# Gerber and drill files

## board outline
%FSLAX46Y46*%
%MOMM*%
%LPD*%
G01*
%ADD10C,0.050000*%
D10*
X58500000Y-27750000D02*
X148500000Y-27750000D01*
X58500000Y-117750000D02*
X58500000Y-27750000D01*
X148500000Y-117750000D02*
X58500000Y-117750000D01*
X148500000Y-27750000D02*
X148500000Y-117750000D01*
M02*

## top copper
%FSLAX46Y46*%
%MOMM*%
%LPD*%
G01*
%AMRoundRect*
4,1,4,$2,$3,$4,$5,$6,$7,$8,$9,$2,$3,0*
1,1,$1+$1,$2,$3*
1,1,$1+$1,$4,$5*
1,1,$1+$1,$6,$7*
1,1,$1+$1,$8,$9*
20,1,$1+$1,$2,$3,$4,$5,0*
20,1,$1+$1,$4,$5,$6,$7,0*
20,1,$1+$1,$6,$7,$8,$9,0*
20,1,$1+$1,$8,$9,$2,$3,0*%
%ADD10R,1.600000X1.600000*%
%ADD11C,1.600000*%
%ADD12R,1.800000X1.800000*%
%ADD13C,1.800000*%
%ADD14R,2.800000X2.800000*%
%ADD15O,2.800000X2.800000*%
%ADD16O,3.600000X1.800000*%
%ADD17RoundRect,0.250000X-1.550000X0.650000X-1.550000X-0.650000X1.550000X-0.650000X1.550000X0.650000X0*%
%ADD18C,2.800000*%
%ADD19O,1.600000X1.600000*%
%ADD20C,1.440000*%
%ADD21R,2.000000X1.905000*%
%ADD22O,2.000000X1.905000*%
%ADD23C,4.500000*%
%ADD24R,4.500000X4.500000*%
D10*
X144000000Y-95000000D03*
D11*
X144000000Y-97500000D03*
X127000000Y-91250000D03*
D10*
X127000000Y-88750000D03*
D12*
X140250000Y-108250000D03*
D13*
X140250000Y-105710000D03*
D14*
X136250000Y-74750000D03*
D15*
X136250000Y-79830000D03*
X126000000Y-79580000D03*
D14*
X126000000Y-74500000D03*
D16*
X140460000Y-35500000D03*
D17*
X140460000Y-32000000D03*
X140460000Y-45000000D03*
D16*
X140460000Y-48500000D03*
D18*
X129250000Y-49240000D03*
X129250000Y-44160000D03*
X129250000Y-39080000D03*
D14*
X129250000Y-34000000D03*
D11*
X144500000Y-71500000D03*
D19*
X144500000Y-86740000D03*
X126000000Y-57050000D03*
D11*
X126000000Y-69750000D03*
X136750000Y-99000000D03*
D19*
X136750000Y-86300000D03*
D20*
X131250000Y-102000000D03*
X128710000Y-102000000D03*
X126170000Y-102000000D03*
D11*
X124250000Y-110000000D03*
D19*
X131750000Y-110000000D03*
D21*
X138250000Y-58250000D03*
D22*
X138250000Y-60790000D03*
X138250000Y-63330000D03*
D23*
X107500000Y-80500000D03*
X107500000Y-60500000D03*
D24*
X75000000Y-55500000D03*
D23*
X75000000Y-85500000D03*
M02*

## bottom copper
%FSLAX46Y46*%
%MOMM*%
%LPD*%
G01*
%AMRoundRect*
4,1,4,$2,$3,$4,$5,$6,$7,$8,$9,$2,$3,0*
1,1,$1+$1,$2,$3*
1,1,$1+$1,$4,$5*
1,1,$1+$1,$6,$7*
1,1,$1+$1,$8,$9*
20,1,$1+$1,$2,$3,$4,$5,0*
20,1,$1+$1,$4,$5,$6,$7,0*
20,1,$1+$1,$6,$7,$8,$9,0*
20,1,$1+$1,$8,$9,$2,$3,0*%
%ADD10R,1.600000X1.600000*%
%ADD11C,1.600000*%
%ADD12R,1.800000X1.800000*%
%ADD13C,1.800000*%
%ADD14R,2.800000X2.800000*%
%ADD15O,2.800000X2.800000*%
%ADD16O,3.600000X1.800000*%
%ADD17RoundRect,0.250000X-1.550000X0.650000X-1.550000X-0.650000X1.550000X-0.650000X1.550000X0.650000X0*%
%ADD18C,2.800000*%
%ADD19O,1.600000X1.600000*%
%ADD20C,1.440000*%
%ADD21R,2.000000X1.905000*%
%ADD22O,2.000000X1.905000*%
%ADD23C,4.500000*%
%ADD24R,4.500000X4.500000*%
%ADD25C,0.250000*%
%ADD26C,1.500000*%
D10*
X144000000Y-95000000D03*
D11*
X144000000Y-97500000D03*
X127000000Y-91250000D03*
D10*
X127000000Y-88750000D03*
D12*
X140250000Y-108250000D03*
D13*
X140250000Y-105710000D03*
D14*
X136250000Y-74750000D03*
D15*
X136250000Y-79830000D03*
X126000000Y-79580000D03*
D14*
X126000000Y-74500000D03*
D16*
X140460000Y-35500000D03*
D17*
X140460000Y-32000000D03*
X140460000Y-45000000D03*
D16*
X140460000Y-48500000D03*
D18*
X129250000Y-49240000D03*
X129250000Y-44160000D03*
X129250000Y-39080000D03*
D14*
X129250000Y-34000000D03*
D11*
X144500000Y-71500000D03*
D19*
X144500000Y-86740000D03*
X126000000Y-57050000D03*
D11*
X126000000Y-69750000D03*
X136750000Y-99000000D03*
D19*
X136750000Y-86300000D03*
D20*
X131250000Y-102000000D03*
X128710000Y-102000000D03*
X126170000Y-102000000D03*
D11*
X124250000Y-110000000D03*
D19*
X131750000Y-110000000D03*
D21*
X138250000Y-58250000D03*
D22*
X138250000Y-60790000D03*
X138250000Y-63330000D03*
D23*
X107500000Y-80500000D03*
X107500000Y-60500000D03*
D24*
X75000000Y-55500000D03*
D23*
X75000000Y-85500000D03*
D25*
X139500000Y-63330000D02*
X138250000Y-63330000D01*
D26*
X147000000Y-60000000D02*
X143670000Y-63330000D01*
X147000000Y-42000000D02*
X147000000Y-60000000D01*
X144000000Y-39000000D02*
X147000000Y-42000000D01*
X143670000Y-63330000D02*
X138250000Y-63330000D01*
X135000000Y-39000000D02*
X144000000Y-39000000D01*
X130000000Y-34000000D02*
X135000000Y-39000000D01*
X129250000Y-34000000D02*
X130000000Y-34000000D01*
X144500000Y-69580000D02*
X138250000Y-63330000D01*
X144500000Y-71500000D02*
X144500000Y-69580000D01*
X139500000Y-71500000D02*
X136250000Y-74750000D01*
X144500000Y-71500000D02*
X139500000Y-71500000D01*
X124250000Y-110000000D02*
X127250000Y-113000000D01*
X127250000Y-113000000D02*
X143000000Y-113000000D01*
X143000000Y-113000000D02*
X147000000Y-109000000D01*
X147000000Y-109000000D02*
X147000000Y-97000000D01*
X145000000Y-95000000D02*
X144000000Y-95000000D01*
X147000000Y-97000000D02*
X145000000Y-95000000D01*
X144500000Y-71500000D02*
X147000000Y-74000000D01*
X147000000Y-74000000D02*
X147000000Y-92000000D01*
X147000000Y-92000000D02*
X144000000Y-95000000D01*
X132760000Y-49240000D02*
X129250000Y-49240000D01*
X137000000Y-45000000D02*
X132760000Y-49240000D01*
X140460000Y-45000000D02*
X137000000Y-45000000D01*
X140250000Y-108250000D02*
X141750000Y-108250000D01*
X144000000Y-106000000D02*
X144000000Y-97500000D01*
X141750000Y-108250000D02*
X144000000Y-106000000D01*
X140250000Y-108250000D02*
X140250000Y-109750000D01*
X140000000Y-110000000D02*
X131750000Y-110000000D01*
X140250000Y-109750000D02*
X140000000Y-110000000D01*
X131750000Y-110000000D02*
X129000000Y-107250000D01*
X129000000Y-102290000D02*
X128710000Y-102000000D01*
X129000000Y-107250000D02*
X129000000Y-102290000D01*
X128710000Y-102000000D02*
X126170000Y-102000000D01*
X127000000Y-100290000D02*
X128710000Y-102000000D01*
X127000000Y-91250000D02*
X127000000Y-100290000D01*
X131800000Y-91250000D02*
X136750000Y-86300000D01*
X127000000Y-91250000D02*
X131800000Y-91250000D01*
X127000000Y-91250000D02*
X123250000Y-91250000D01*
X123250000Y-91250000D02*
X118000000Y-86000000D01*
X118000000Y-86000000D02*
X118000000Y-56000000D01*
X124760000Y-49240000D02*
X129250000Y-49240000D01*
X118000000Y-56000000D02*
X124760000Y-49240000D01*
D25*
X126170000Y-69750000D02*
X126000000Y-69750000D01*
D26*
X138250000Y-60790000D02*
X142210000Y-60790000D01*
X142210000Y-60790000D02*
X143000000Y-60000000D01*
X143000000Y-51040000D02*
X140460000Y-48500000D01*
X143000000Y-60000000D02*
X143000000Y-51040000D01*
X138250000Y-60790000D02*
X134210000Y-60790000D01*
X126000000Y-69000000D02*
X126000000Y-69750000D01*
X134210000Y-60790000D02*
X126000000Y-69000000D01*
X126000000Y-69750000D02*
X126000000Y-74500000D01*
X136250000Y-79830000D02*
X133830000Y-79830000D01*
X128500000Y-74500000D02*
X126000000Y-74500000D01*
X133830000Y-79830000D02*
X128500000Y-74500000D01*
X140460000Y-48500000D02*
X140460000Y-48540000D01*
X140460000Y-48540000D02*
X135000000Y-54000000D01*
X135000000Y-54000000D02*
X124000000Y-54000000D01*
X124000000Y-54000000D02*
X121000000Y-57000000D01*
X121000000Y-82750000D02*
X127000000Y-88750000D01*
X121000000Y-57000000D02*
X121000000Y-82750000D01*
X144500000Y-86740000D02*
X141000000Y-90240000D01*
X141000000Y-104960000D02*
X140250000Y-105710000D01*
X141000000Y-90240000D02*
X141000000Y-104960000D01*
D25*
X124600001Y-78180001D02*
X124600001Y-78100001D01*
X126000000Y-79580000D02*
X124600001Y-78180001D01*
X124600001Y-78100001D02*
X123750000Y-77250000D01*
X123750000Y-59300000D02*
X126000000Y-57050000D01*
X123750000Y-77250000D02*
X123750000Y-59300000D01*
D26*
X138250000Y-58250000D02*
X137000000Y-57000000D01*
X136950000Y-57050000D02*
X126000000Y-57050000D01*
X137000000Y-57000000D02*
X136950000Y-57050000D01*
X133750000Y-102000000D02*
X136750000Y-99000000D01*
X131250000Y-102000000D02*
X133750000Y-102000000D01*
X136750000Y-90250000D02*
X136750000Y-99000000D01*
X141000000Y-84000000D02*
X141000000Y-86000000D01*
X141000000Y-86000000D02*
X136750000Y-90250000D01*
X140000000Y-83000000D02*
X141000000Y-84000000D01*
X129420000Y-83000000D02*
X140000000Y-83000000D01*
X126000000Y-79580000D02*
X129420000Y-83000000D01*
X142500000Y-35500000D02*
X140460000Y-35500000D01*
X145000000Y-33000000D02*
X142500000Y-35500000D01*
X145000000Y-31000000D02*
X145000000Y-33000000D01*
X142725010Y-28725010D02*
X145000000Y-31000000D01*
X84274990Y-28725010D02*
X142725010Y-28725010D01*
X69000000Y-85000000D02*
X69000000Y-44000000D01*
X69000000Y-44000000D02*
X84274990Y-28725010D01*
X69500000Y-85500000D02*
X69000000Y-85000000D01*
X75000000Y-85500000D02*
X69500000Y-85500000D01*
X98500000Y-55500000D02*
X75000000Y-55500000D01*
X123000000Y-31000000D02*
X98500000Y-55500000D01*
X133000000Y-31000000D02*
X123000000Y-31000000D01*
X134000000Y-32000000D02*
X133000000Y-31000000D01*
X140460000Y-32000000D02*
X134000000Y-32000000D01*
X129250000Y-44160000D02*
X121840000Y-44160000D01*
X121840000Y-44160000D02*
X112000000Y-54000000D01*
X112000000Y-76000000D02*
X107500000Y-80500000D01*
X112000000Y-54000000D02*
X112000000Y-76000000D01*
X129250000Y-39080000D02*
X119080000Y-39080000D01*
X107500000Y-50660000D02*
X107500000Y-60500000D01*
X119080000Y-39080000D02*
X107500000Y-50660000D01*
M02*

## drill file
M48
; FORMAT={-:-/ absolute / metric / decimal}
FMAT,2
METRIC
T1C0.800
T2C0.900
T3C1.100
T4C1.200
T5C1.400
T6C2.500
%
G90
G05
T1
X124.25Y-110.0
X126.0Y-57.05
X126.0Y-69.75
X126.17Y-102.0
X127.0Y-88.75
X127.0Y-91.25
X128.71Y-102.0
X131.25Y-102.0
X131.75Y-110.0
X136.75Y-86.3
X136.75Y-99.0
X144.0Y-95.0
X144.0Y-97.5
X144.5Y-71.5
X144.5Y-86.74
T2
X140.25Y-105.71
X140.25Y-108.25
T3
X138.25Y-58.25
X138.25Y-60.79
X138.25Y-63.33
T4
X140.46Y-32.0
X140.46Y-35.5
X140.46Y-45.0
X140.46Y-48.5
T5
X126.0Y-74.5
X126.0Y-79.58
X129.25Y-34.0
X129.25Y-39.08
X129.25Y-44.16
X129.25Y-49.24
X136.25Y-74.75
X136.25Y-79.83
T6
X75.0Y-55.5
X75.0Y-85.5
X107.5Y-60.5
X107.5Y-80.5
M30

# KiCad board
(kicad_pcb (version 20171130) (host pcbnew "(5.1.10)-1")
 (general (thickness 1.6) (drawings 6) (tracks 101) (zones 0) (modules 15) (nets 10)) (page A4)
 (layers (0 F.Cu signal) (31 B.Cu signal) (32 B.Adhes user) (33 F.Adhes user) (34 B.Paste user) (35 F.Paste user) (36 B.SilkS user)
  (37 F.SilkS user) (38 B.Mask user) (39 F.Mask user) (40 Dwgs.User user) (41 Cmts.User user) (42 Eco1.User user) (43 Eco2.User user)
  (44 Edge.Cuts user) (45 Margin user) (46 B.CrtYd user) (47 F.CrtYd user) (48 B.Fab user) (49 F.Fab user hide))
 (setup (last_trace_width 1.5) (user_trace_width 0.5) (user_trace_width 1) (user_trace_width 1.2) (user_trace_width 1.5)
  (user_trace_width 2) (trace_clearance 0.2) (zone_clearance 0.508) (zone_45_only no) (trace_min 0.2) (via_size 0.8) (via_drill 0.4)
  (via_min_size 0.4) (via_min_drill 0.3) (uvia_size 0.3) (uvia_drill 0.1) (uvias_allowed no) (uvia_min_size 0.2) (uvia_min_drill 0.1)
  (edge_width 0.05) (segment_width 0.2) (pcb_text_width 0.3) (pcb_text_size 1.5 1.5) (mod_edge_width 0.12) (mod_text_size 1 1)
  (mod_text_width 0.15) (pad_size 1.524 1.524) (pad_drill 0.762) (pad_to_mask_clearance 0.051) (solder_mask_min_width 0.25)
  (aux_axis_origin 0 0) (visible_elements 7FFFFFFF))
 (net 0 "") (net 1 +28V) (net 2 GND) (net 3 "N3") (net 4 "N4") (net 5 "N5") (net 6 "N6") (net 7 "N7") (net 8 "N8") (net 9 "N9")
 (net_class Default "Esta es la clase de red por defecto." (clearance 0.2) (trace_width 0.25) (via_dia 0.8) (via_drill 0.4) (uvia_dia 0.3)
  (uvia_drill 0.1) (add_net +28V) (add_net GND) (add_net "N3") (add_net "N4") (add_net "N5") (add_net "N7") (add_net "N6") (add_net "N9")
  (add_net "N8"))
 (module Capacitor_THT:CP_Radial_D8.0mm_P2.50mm (layer F.Cu) (at 144 95 270)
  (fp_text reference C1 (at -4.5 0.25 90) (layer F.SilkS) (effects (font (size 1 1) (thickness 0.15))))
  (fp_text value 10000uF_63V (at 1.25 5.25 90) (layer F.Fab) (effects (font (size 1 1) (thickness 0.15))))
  (pad 1 thru_hole rect (at 0 0 270) (size 1.6 1.6) (drill 0.8) (layers *.Cu *.Mask) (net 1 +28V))
  (pad 2 thru_hole circle (at 2.5 0 270) (size 1.6 1.6) (drill 0.8) (layers *.Cu *.Mask) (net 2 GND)))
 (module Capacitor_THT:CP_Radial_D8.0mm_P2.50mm (layer F.Cu) (at 127 88.75 270)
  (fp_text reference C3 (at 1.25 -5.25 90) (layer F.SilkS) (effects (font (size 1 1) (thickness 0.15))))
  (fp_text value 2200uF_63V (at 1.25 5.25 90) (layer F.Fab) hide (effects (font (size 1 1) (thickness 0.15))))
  (pad 2 thru_hole circle (at 2.5 0 270) (size 1.6 1.6) (drill 0.8) (layers *.Cu *.Mask) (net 2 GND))
  (pad 1 thru_hole rect (at 0 0 270) (size 1.6 1.6) (drill 0.8) (layers *.Cu *.Mask) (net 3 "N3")))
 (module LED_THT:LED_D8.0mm (layer F.Cu) (at 140.25 108.25 90)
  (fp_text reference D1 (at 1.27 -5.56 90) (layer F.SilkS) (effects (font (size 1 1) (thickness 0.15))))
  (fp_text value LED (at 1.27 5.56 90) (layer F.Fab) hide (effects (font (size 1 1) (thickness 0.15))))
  (pad 1 thru_hole rect (at 0 0 90) (size 1.8 1.8) (drill 0.9) (layers *.Cu *.Mask) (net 2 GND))
  (pad 2 thru_hole circle (at 2.54 0 90) (size 1.8 1.8) (drill 0.9) (layers *.Cu *.Mask) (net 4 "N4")))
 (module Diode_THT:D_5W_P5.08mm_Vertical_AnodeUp (layer F.Cu) (at 136.25 74.75 270)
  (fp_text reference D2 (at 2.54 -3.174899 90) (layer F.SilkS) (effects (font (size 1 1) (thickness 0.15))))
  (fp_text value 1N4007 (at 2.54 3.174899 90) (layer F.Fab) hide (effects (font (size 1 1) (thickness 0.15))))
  (pad 1 thru_hole rect (at 0 0 270) (size 2.8 2.8) (drill 1.4) (layers *.Cu *.Mask) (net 1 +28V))
  (pad 2 thru_hole oval (at 5.08 0 270) (size 2.8 2.8) (drill 1.4) (layers *.Cu *.Mask) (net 3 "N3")))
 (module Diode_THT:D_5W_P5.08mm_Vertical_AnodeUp (layer F.Cu) (at 126 74.5 270)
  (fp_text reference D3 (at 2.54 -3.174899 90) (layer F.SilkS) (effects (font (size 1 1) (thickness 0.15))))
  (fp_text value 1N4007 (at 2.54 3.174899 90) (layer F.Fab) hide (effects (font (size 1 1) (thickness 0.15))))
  (pad 2 thru_hole oval (at 5.08 0 270) (size 2.8 2.8) (drill 1.4) (layers *.Cu *.Mask) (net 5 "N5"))
  (pad 1 thru_hole rect (at 0 0 270) (size 2.8 2.8) (drill 1.4) (layers *.Cu *.Mask) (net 3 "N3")))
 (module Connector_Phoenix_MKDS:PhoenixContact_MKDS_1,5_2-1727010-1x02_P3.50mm (layer F.Cu) (at 143 32 270)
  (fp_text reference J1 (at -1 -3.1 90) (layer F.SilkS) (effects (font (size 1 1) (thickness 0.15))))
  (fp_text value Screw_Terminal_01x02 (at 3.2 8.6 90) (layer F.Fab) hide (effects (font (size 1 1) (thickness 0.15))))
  (pad 2 thru_hole oval (at 3.5 2.54 270) (size 1.8 3.6) (drill 1.2) (layers *.Cu *.Mask) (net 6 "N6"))
  (pad 1 thru_hole roundrect (at 0 2.54 270) (size 1.8 3.6) (drill 1.2) (layers *.Cu *.Mask) (roundrect_rratio 0.138889) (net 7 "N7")))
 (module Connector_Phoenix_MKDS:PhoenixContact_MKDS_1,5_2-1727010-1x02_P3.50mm (layer F.Cu) (at 143 45 270)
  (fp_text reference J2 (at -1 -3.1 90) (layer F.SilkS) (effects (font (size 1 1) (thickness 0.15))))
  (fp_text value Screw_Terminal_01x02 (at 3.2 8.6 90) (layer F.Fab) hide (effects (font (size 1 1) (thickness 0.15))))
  (pad 1 thru_hole roundrect (at 0 2.54 270) (size 1.8 3.6) (drill 1.2) (layers *.Cu *.Mask) (roundrect_rratio 0.138889) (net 2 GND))
  (pad 2 thru_hole oval (at 3.5 2.54 270) (size 1.8 3.6) (drill 1.2) (layers *.Cu *.Mask) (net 3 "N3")))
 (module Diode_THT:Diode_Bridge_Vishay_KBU (layer F.Cu) (at 129.25 34 270)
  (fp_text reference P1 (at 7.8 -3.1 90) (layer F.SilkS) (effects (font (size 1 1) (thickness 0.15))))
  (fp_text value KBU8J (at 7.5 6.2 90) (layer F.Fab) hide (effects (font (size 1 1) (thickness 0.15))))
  (pad 4 thru_hole circle (at 15.24 0 270) (size 2.8 2.8) (drill 1.4) (layers *.Cu *.Mask) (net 2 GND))
  (pad 3 thru_hole circle (at 10.16 0 270) (size 2.8 2.8) (drill 1.4) (layers *.Cu *.Mask) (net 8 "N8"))
  (pad 2 thru_hole circle (at 5.08 0 270) (size 2.8 2.8) (drill 1.4) (layers *.Cu *.Mask) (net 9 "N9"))
  (pad 1 thru_hole rect (at 0 0 270) (size 2.8 2.8) (drill 1.4) (layers *.Cu *.Mask) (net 1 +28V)))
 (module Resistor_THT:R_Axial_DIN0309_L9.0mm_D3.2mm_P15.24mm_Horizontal (layer F.Cu) (at 144.5 71.5 270)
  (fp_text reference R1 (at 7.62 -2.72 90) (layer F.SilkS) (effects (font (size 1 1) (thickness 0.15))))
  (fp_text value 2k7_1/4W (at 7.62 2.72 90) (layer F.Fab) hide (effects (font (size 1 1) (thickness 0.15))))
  (pad 1 thru_hole circle (at 0 0 270) (size 1.6 1.6) (drill 0.8) (layers *.Cu *.Mask) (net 1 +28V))
  (pad 2 thru_hole oval (at 15.24 0 270) (size 1.6 1.6) (drill 0.8) (layers *.Cu *.Mask) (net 4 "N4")))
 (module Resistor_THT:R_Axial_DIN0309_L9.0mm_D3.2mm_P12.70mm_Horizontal (layer F.Cu) (at 126 69.75 90)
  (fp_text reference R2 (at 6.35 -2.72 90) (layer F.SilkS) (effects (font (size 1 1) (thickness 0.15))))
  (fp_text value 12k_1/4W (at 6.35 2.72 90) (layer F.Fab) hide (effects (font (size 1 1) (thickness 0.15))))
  (pad 2 thru_hole oval (at 12.7 0 90) (size 1.6 1.6) (drill 0.8) (layers *.Cu *.Mask) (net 5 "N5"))
  (pad 1 thru_hole circle (at 0 0 90) (size 1.6 1.6) (drill 0.8) (layers *.Cu *.Mask) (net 3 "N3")))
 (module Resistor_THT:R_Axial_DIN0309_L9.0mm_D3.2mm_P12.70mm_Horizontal (layer F.Cu) (at 136.75 99 90)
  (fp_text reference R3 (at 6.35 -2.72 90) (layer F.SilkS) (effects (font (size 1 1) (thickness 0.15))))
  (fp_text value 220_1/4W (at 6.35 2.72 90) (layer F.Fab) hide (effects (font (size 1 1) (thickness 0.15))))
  (pad 1 thru_hole circle (at 0 0 90) (size 1.6 1.6) (drill 0.8) (layers *.Cu *.Mask) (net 5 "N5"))
  (pad 2 thru_hole oval (at 12.7 0 90) (size 1.6 1.6) (drill 0.8) (layers *.Cu *.Mask) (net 2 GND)))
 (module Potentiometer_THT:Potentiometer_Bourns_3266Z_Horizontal (layer F.Cu) (at 131.25 102)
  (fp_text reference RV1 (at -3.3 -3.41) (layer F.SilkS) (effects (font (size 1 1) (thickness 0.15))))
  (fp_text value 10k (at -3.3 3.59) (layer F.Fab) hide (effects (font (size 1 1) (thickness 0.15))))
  (pad 1 thru_hole circle (at 0 0) (size 1.44 1.44) (drill 0.8) (layers *.Cu *.Mask) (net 5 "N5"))
  (pad 2 thru_hole circle (at -2.54 0) (size 1.44 1.44) (drill 0.8) (layers *.Cu *.Mask) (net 2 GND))
  (pad 3 thru_hole circle (at -5.08 0) (size 1.44 1.44) (drill 0.8) (layers *.Cu *.Mask) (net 2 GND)))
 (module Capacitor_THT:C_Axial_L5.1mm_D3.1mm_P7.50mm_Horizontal (layer F.Cu) (at 124.25 110)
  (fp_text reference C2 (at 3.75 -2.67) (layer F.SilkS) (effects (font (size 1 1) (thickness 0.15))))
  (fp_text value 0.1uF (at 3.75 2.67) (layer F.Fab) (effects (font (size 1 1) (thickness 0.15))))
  (pad 1 thru_hole circle (at 0 0) (size 1.6 1.6) (drill 0.8) (layers *.Cu *.Mask) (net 1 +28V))
  (pad 2 thru_hole oval (at 7.5 0) (size 1.6 1.6) (drill 0.8) (layers *.Cu *.Mask) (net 2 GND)))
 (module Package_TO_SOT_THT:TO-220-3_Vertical (layer F.Cu) (at 138.25 58.25 270)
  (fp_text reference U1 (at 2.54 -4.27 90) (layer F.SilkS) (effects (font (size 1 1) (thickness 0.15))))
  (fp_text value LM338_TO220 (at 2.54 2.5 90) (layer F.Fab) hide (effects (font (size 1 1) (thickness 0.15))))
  (pad 1 thru_hole rect (at 0 0 270) (size 1.905 2) (drill 1.1) (layers *.Cu *.Mask) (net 5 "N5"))
  (pad 2 thru_hole oval (at 2.54 0 270) (size 1.905 2) (drill 1.1) (layers *.Cu *.Mask) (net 3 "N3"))
  (pad 3 thru_hole oval (at 5.08 0 270) (size 1.905 2) (drill 1.1) (layers *.Cu *.Mask) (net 1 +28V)))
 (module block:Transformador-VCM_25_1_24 (layer F.Cu) (at 75 55.5 270)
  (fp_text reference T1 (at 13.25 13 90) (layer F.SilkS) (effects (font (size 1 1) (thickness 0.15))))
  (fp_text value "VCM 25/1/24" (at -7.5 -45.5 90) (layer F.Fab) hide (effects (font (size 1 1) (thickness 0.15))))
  (pad 4 thru_hole circle (at 25 -32.5 270) (size 4.5 4.5) (drill 2.5) (layers *.Cu *.Mask) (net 8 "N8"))
  (pad 3 thru_hole circle (at 5 -32.5 270) (size 4.5 4.5) (drill 2.5) (layers *.Cu *.Mask) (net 9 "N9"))
  (pad 1 thru_hole rect (at 0 0 270) (size 4.5 4.5) (drill 2.5) (layers *.Cu *.Mask) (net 7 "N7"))
  (pad 2 thru_hole circle (at 30 0 270) (size 4.5 4.5) (drill 2.5) (layers *.Cu *.Mask) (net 6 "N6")))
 (gr_line (start 58.5 27.75) (end 148.5 27.75) (layer Edge.Cuts) (width 0.05))
 (gr_line (start 58.5 117.75) (end 58.5 27.75) (layer Edge.Cuts) (width 0.05))
 (gr_line (start 148.5 117.75) (end 58.5 117.75) (layer Edge.Cuts) (width 0.05))
 (gr_line (start 148.5 27.75) (end 148.5 117.75) (layer Edge.Cuts) (width 0.05))
 (segment (start 139.5 63.33) (end 138.25 63.33) (width 0.25) (layer B.Cu) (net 1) (status 20))
 (segment (start 147 60) (end 143.67 63.33) (width 1.5) (layer B.Cu) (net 1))
 (segment (start 147 42) (end 147 60) (width 1.5) (layer B.Cu) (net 1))
 (segment (start 144 39) (end 147 42) (width 1.5) (layer B.Cu) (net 1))
 (segment (start 143.67 63.33) (end 138.25 63.33) (width 1.5) (layer B.Cu) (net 1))
 (segment (start 135 39) (end 144 39) (width 1.5) (layer B.Cu) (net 1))
 (segment (start 130 34) (end 135 39) (width 1.5) (layer B.Cu) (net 1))
 (segment (start 129.25 34) (end 130 34) (width 1.5) (layer B.Cu) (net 1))
 (segment (start 144.5 69.58) (end 138.25 63.33) (width 1.5) (layer B.Cu) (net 1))
 (segment (start 144.5 71.5) (end 144.5 69.58) (width 1.5) (layer B.Cu) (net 1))
 (segment (start 139.5 71.5) (end 136.25 74.75) (width 1.5) (layer B.Cu) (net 1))
 (segment (start 144.5 71.5) (end 139.5 71.5) (width 1.5) (layer B.Cu) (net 1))
 (segment (start 124.25 110) (end 127.25 113) (width 1.5) (layer B.Cu) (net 1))
 (segment (start 127.25 113) (end 143 113) (width 1.5) (layer B.Cu) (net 1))
 (segment (start 143 113) (end 147 109) (width 1.5) (layer B.Cu) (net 1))
 (segment (start 147 109) (end 147 97) (width 1.5) (layer B.Cu) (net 1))
 (segment (start 145 95) (end 144 95) (width 1.5) (layer B.Cu) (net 1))
 (segment (start 147 97) (end 145 95) (width 1.5) (layer B.Cu) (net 1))
 (segment (start 144.5 71.5) (end 147 74) (width 1.5) (layer B.Cu) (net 1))
 (segment (start 147 74) (end 147 92) (width 1.5) (layer B.Cu) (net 1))
 (segment (start 147 92) (end 144 95) (width 1.5) (layer B.Cu) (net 1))
 (segment (start 132.76 49.24) (end 129.25 49.24) (width 1.5) (layer B.Cu) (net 2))
 (segment (start 137 45) (end 132.76 49.24) (width 1.5) (layer B.Cu) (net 2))
 (segment (start 140.46 45) (end 137 45) (width 1.5) (layer B.Cu) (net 2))
 (segment (start 140.25 108.25) (end 141.75 108.25) (width 1.5) (layer B.Cu) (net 2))
 (segment (start 144 106) (end 144 97.5) (width 1.5) (layer B.Cu) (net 2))
 (segment (start 141.75 108.25) (end 144 106) (width 1.5) (layer B.Cu) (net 2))
 (segment (start 140.25 108.25) (end 140.25 109.75) (width 1.5) (layer B.Cu) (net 2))
 (segment (start 140 110) (end 131.75 110) (width 1.5) (layer B.Cu) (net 2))
 (segment (start 140.25 109.75) (end 140 110) (width 1.5) (layer B.Cu) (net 2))
 (segment (start 131.75 110) (end 129 107.25) (width 1.5) (layer B.Cu) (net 2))
 (segment (start 129 102.29) (end 128.71 102) (width 1.5) (layer B.Cu) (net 2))
 (segment (start 129 107.25) (end 129 102.29) (width 1.5) (layer B.Cu) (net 2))
 (segment (start 128.71 102) (end 126.17 102) (width 1.5) (layer B.Cu) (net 2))
 (segment (start 127 100.29) (end 128.71 102) (width 1.5) (layer B.Cu) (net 2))
 (segment (start 127 91.25) (end 127 100.29) (width 1.5) (layer B.Cu) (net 2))
 (segment (start 131.8 91.25) (end 136.75 86.3) (width 1.5) (layer B.Cu) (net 2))
 (segment (start 127 91.25) (end 131.8 91.25) (width 1.5) (layer B.Cu) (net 2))
 (segment (start 127 91.25) (end 123.25 91.25) (width 1.5) (layer B.Cu) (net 2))
 (segment (start 123.25 91.25) (end 118 86) (width 1.5) (layer B.Cu) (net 2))
 (segment (start 118 86) (end 118 56) (width 1.5) (layer B.Cu) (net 2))
 (segment (start 124.76 49.24) (end 129.25 49.24) (width 1.5) (layer B.Cu) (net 2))
 (segment (start 118 56) (end 124.76 49.24) (width 1.5) (layer B.Cu) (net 2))
 (segment (start 126.17 69.75) (end 126 69.75) (width 0.25) (layer B.Cu) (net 3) (status 30))
 (segment (start 138.25 60.79) (end 142.21 60.79) (width 1.5) (layer B.Cu) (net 3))
 (segment (start 142.21 60.79) (end 143 60) (width 1.5) (layer B.Cu) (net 3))
 (segment (start 143 51.04) (end 140.46 48.5) (width 1.5) (layer B.Cu) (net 3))
 (segment (start 143 60) (end 143 51.04) (width 1.5) (layer B.Cu) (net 3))
 (segment (start 138.25 60.79) (end 134.21 60.79) (width 1.5) (layer B.Cu) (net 3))
 (segment (start 126 69) (end 126 69.75) (width 1.5) (layer B.Cu) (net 3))
 (segment (start 134.21 60.79) (end 126 69) (width 1.5) (layer B.Cu) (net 3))
 (segment (start 126 69.75) (end 126 74.5) (width 1.5) (layer B.Cu) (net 3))
 (segment (start 136.25 79.83) (end 133.83 79.83) (width 1.5) (layer B.Cu) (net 3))
 (segment (start 128.5 74.5) (end 126 74.5) (width 1.5) (layer B.Cu) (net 3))
 (segment (start 133.83 79.83) (end 128.5 74.5) (width 1.5) (layer B.Cu) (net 3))
 (segment (start 140.46 48.5) (end 140.46 48.54) (width 1.5) (layer B.Cu) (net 3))
 (segment (start 140.46 48.54) (end 135 54) (width 1.5) (layer B.Cu) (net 3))
 (segment (start 135 54) (end 124 54) (width 1.5) (layer B.Cu) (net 3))
 (segment (start 124 54) (end 121 57) (width 1.5) (layer B.Cu) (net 3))
 (segment (start 121 82.75) (end 127 88.75) (width 1.5) (layer B.Cu) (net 3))
 (segment (start 121 57) (end 121 82.75) (width 1.5) (layer B.Cu) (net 3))
 (segment (start 144.5 86.74) (end 141 90.24) (width 1.5) (layer B.Cu) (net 4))
 (segment (start 141 104.96) (end 140.25 105.71) (width 1.5) (layer B.Cu) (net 4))
 (segment (start 141 90.24) (end 141 104.96) (width 1.5) (layer B.Cu) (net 4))
 (segment (start 124.600001 78.180001) (end 124.600001 78.100001) (width 0.25) (layer B.Cu) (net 5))
 (segment (start 126 79.58) (end 124.600001 78.180001) (width 0.25) (layer B.Cu) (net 5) (status 10))
 (segment (start 124.600001 78.100001) (end 123.75 77.25) (width 0.25) (layer B.Cu) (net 5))
 (segment (start 123.75 59.3) (end 126 57.05) (width 0.25) (layer B.Cu) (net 5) (status 20))
 (segment (start 123.75 77.25) (end 123.75 59.3) (width 0.25) (layer B.Cu) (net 5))
 (segment (start 138.25 58.25) (end 137 57) (width 1.5) (layer B.Cu) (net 5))
 (segment (start 136.95 57.05) (end 126 57.05) (width 1.5) (layer B.Cu) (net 5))
 (segment (start 137 57) (end 136.95 57.05) (width 1.5) (layer B.Cu) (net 5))
 (segment (start 133.75 102) (end 136.75 99) (width 1.5) (layer B.Cu) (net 5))
 (segment (start 131.25 102) (end 133.75 102) (width 1.5) (layer B.Cu) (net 5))
 (segment (start 136.75 90.25) (end 136.75 99) (width 1.5) (layer B.Cu) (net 5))
 (segment (start 141 84) (end 141 86) (width 1.5) (layer B.Cu) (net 5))
 (segment (start 141 86) (end 136.75 90.25) (width 1.5) (layer B.Cu) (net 5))
 (segment (start 140 83) (end 141 84) (width 1.5) (layer B.Cu) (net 5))
 (segment (start 129.42 83) (end 140 83) (width 1.5) (layer B.Cu) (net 5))
 (segment (start 126 79.58) (end 129.42 83) (width 1.5) (layer B.Cu) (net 5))
 (segment (start 142.5 35.5) (end 140.46 35.5) (width 1.5) (layer B.Cu) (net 6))
 (segment (start 145 33) (end 142.5 35.5) (width 1.5) (layer B.Cu) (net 6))
 (segment (start 145 31) (end 145 33) (width 1.5) (layer B.Cu) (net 6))
 (segment (start 142.72501 28.72501) (end 145 31) (width 1.5) (layer B.Cu) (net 6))
 (segment (start 84.27499 28.72501) (end 142.72501 28.72501) (width 1.5) (layer B.Cu) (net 6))
 (segment (start 69 85) (end 69 44) (width 1.5) (layer B.Cu) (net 6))
 (segment (start 69 44) (end 84.27499 28.72501) (width 1.5) (layer B.Cu) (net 6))
 (segment (start 69.5 85.5) (end 69 85) (width 1.5) (layer B.Cu) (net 6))
 (segment (start 75 85.5) (end 69.5 85.5) (width 1.5) (layer B.Cu) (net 6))
 (segment (start 98.5 55.5) (end 75 55.5) (width 1.5) (layer B.Cu) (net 7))
 (segment (start 123 31) (end 98.5 55.5) (width 1.5) (layer B.Cu) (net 7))
 (segment (start 133 31) (end 123 31) (width 1.5) (layer B.Cu) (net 7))
 (segment (start 134 32) (end 133 31) (width 1.5) (layer B.Cu) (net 7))
 (segment (start 140.46 32) (end 134 32) (width 1.5) (layer B.Cu) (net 7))
 (segment (start 129.25 44.16) (end 121.84 44.16) (width 1.5) (layer B.Cu) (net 8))
 (segment (start 121.84 44.16) (end 112 54) (width 1.5) (layer B.Cu) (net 8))
 (segment (start 112 76) (end 107.5 80.5) (width 1.5) (layer B.Cu) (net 8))
 (segment (start 112 54) (end 112 76) (width 1.5) (layer B.Cu) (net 8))
 (segment (start 129.25 39.08) (end 119.08 39.08) (width 1.5) (layer B.Cu) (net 9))
 (segment (start 107.5 50.66) (end 107.5 60.5) (width 1.5) (layer B.Cu) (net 9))
 (segment (start 119.08 39.08) (end 107.5 50.66) (width 1.5) (layer B.Cu) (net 9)))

